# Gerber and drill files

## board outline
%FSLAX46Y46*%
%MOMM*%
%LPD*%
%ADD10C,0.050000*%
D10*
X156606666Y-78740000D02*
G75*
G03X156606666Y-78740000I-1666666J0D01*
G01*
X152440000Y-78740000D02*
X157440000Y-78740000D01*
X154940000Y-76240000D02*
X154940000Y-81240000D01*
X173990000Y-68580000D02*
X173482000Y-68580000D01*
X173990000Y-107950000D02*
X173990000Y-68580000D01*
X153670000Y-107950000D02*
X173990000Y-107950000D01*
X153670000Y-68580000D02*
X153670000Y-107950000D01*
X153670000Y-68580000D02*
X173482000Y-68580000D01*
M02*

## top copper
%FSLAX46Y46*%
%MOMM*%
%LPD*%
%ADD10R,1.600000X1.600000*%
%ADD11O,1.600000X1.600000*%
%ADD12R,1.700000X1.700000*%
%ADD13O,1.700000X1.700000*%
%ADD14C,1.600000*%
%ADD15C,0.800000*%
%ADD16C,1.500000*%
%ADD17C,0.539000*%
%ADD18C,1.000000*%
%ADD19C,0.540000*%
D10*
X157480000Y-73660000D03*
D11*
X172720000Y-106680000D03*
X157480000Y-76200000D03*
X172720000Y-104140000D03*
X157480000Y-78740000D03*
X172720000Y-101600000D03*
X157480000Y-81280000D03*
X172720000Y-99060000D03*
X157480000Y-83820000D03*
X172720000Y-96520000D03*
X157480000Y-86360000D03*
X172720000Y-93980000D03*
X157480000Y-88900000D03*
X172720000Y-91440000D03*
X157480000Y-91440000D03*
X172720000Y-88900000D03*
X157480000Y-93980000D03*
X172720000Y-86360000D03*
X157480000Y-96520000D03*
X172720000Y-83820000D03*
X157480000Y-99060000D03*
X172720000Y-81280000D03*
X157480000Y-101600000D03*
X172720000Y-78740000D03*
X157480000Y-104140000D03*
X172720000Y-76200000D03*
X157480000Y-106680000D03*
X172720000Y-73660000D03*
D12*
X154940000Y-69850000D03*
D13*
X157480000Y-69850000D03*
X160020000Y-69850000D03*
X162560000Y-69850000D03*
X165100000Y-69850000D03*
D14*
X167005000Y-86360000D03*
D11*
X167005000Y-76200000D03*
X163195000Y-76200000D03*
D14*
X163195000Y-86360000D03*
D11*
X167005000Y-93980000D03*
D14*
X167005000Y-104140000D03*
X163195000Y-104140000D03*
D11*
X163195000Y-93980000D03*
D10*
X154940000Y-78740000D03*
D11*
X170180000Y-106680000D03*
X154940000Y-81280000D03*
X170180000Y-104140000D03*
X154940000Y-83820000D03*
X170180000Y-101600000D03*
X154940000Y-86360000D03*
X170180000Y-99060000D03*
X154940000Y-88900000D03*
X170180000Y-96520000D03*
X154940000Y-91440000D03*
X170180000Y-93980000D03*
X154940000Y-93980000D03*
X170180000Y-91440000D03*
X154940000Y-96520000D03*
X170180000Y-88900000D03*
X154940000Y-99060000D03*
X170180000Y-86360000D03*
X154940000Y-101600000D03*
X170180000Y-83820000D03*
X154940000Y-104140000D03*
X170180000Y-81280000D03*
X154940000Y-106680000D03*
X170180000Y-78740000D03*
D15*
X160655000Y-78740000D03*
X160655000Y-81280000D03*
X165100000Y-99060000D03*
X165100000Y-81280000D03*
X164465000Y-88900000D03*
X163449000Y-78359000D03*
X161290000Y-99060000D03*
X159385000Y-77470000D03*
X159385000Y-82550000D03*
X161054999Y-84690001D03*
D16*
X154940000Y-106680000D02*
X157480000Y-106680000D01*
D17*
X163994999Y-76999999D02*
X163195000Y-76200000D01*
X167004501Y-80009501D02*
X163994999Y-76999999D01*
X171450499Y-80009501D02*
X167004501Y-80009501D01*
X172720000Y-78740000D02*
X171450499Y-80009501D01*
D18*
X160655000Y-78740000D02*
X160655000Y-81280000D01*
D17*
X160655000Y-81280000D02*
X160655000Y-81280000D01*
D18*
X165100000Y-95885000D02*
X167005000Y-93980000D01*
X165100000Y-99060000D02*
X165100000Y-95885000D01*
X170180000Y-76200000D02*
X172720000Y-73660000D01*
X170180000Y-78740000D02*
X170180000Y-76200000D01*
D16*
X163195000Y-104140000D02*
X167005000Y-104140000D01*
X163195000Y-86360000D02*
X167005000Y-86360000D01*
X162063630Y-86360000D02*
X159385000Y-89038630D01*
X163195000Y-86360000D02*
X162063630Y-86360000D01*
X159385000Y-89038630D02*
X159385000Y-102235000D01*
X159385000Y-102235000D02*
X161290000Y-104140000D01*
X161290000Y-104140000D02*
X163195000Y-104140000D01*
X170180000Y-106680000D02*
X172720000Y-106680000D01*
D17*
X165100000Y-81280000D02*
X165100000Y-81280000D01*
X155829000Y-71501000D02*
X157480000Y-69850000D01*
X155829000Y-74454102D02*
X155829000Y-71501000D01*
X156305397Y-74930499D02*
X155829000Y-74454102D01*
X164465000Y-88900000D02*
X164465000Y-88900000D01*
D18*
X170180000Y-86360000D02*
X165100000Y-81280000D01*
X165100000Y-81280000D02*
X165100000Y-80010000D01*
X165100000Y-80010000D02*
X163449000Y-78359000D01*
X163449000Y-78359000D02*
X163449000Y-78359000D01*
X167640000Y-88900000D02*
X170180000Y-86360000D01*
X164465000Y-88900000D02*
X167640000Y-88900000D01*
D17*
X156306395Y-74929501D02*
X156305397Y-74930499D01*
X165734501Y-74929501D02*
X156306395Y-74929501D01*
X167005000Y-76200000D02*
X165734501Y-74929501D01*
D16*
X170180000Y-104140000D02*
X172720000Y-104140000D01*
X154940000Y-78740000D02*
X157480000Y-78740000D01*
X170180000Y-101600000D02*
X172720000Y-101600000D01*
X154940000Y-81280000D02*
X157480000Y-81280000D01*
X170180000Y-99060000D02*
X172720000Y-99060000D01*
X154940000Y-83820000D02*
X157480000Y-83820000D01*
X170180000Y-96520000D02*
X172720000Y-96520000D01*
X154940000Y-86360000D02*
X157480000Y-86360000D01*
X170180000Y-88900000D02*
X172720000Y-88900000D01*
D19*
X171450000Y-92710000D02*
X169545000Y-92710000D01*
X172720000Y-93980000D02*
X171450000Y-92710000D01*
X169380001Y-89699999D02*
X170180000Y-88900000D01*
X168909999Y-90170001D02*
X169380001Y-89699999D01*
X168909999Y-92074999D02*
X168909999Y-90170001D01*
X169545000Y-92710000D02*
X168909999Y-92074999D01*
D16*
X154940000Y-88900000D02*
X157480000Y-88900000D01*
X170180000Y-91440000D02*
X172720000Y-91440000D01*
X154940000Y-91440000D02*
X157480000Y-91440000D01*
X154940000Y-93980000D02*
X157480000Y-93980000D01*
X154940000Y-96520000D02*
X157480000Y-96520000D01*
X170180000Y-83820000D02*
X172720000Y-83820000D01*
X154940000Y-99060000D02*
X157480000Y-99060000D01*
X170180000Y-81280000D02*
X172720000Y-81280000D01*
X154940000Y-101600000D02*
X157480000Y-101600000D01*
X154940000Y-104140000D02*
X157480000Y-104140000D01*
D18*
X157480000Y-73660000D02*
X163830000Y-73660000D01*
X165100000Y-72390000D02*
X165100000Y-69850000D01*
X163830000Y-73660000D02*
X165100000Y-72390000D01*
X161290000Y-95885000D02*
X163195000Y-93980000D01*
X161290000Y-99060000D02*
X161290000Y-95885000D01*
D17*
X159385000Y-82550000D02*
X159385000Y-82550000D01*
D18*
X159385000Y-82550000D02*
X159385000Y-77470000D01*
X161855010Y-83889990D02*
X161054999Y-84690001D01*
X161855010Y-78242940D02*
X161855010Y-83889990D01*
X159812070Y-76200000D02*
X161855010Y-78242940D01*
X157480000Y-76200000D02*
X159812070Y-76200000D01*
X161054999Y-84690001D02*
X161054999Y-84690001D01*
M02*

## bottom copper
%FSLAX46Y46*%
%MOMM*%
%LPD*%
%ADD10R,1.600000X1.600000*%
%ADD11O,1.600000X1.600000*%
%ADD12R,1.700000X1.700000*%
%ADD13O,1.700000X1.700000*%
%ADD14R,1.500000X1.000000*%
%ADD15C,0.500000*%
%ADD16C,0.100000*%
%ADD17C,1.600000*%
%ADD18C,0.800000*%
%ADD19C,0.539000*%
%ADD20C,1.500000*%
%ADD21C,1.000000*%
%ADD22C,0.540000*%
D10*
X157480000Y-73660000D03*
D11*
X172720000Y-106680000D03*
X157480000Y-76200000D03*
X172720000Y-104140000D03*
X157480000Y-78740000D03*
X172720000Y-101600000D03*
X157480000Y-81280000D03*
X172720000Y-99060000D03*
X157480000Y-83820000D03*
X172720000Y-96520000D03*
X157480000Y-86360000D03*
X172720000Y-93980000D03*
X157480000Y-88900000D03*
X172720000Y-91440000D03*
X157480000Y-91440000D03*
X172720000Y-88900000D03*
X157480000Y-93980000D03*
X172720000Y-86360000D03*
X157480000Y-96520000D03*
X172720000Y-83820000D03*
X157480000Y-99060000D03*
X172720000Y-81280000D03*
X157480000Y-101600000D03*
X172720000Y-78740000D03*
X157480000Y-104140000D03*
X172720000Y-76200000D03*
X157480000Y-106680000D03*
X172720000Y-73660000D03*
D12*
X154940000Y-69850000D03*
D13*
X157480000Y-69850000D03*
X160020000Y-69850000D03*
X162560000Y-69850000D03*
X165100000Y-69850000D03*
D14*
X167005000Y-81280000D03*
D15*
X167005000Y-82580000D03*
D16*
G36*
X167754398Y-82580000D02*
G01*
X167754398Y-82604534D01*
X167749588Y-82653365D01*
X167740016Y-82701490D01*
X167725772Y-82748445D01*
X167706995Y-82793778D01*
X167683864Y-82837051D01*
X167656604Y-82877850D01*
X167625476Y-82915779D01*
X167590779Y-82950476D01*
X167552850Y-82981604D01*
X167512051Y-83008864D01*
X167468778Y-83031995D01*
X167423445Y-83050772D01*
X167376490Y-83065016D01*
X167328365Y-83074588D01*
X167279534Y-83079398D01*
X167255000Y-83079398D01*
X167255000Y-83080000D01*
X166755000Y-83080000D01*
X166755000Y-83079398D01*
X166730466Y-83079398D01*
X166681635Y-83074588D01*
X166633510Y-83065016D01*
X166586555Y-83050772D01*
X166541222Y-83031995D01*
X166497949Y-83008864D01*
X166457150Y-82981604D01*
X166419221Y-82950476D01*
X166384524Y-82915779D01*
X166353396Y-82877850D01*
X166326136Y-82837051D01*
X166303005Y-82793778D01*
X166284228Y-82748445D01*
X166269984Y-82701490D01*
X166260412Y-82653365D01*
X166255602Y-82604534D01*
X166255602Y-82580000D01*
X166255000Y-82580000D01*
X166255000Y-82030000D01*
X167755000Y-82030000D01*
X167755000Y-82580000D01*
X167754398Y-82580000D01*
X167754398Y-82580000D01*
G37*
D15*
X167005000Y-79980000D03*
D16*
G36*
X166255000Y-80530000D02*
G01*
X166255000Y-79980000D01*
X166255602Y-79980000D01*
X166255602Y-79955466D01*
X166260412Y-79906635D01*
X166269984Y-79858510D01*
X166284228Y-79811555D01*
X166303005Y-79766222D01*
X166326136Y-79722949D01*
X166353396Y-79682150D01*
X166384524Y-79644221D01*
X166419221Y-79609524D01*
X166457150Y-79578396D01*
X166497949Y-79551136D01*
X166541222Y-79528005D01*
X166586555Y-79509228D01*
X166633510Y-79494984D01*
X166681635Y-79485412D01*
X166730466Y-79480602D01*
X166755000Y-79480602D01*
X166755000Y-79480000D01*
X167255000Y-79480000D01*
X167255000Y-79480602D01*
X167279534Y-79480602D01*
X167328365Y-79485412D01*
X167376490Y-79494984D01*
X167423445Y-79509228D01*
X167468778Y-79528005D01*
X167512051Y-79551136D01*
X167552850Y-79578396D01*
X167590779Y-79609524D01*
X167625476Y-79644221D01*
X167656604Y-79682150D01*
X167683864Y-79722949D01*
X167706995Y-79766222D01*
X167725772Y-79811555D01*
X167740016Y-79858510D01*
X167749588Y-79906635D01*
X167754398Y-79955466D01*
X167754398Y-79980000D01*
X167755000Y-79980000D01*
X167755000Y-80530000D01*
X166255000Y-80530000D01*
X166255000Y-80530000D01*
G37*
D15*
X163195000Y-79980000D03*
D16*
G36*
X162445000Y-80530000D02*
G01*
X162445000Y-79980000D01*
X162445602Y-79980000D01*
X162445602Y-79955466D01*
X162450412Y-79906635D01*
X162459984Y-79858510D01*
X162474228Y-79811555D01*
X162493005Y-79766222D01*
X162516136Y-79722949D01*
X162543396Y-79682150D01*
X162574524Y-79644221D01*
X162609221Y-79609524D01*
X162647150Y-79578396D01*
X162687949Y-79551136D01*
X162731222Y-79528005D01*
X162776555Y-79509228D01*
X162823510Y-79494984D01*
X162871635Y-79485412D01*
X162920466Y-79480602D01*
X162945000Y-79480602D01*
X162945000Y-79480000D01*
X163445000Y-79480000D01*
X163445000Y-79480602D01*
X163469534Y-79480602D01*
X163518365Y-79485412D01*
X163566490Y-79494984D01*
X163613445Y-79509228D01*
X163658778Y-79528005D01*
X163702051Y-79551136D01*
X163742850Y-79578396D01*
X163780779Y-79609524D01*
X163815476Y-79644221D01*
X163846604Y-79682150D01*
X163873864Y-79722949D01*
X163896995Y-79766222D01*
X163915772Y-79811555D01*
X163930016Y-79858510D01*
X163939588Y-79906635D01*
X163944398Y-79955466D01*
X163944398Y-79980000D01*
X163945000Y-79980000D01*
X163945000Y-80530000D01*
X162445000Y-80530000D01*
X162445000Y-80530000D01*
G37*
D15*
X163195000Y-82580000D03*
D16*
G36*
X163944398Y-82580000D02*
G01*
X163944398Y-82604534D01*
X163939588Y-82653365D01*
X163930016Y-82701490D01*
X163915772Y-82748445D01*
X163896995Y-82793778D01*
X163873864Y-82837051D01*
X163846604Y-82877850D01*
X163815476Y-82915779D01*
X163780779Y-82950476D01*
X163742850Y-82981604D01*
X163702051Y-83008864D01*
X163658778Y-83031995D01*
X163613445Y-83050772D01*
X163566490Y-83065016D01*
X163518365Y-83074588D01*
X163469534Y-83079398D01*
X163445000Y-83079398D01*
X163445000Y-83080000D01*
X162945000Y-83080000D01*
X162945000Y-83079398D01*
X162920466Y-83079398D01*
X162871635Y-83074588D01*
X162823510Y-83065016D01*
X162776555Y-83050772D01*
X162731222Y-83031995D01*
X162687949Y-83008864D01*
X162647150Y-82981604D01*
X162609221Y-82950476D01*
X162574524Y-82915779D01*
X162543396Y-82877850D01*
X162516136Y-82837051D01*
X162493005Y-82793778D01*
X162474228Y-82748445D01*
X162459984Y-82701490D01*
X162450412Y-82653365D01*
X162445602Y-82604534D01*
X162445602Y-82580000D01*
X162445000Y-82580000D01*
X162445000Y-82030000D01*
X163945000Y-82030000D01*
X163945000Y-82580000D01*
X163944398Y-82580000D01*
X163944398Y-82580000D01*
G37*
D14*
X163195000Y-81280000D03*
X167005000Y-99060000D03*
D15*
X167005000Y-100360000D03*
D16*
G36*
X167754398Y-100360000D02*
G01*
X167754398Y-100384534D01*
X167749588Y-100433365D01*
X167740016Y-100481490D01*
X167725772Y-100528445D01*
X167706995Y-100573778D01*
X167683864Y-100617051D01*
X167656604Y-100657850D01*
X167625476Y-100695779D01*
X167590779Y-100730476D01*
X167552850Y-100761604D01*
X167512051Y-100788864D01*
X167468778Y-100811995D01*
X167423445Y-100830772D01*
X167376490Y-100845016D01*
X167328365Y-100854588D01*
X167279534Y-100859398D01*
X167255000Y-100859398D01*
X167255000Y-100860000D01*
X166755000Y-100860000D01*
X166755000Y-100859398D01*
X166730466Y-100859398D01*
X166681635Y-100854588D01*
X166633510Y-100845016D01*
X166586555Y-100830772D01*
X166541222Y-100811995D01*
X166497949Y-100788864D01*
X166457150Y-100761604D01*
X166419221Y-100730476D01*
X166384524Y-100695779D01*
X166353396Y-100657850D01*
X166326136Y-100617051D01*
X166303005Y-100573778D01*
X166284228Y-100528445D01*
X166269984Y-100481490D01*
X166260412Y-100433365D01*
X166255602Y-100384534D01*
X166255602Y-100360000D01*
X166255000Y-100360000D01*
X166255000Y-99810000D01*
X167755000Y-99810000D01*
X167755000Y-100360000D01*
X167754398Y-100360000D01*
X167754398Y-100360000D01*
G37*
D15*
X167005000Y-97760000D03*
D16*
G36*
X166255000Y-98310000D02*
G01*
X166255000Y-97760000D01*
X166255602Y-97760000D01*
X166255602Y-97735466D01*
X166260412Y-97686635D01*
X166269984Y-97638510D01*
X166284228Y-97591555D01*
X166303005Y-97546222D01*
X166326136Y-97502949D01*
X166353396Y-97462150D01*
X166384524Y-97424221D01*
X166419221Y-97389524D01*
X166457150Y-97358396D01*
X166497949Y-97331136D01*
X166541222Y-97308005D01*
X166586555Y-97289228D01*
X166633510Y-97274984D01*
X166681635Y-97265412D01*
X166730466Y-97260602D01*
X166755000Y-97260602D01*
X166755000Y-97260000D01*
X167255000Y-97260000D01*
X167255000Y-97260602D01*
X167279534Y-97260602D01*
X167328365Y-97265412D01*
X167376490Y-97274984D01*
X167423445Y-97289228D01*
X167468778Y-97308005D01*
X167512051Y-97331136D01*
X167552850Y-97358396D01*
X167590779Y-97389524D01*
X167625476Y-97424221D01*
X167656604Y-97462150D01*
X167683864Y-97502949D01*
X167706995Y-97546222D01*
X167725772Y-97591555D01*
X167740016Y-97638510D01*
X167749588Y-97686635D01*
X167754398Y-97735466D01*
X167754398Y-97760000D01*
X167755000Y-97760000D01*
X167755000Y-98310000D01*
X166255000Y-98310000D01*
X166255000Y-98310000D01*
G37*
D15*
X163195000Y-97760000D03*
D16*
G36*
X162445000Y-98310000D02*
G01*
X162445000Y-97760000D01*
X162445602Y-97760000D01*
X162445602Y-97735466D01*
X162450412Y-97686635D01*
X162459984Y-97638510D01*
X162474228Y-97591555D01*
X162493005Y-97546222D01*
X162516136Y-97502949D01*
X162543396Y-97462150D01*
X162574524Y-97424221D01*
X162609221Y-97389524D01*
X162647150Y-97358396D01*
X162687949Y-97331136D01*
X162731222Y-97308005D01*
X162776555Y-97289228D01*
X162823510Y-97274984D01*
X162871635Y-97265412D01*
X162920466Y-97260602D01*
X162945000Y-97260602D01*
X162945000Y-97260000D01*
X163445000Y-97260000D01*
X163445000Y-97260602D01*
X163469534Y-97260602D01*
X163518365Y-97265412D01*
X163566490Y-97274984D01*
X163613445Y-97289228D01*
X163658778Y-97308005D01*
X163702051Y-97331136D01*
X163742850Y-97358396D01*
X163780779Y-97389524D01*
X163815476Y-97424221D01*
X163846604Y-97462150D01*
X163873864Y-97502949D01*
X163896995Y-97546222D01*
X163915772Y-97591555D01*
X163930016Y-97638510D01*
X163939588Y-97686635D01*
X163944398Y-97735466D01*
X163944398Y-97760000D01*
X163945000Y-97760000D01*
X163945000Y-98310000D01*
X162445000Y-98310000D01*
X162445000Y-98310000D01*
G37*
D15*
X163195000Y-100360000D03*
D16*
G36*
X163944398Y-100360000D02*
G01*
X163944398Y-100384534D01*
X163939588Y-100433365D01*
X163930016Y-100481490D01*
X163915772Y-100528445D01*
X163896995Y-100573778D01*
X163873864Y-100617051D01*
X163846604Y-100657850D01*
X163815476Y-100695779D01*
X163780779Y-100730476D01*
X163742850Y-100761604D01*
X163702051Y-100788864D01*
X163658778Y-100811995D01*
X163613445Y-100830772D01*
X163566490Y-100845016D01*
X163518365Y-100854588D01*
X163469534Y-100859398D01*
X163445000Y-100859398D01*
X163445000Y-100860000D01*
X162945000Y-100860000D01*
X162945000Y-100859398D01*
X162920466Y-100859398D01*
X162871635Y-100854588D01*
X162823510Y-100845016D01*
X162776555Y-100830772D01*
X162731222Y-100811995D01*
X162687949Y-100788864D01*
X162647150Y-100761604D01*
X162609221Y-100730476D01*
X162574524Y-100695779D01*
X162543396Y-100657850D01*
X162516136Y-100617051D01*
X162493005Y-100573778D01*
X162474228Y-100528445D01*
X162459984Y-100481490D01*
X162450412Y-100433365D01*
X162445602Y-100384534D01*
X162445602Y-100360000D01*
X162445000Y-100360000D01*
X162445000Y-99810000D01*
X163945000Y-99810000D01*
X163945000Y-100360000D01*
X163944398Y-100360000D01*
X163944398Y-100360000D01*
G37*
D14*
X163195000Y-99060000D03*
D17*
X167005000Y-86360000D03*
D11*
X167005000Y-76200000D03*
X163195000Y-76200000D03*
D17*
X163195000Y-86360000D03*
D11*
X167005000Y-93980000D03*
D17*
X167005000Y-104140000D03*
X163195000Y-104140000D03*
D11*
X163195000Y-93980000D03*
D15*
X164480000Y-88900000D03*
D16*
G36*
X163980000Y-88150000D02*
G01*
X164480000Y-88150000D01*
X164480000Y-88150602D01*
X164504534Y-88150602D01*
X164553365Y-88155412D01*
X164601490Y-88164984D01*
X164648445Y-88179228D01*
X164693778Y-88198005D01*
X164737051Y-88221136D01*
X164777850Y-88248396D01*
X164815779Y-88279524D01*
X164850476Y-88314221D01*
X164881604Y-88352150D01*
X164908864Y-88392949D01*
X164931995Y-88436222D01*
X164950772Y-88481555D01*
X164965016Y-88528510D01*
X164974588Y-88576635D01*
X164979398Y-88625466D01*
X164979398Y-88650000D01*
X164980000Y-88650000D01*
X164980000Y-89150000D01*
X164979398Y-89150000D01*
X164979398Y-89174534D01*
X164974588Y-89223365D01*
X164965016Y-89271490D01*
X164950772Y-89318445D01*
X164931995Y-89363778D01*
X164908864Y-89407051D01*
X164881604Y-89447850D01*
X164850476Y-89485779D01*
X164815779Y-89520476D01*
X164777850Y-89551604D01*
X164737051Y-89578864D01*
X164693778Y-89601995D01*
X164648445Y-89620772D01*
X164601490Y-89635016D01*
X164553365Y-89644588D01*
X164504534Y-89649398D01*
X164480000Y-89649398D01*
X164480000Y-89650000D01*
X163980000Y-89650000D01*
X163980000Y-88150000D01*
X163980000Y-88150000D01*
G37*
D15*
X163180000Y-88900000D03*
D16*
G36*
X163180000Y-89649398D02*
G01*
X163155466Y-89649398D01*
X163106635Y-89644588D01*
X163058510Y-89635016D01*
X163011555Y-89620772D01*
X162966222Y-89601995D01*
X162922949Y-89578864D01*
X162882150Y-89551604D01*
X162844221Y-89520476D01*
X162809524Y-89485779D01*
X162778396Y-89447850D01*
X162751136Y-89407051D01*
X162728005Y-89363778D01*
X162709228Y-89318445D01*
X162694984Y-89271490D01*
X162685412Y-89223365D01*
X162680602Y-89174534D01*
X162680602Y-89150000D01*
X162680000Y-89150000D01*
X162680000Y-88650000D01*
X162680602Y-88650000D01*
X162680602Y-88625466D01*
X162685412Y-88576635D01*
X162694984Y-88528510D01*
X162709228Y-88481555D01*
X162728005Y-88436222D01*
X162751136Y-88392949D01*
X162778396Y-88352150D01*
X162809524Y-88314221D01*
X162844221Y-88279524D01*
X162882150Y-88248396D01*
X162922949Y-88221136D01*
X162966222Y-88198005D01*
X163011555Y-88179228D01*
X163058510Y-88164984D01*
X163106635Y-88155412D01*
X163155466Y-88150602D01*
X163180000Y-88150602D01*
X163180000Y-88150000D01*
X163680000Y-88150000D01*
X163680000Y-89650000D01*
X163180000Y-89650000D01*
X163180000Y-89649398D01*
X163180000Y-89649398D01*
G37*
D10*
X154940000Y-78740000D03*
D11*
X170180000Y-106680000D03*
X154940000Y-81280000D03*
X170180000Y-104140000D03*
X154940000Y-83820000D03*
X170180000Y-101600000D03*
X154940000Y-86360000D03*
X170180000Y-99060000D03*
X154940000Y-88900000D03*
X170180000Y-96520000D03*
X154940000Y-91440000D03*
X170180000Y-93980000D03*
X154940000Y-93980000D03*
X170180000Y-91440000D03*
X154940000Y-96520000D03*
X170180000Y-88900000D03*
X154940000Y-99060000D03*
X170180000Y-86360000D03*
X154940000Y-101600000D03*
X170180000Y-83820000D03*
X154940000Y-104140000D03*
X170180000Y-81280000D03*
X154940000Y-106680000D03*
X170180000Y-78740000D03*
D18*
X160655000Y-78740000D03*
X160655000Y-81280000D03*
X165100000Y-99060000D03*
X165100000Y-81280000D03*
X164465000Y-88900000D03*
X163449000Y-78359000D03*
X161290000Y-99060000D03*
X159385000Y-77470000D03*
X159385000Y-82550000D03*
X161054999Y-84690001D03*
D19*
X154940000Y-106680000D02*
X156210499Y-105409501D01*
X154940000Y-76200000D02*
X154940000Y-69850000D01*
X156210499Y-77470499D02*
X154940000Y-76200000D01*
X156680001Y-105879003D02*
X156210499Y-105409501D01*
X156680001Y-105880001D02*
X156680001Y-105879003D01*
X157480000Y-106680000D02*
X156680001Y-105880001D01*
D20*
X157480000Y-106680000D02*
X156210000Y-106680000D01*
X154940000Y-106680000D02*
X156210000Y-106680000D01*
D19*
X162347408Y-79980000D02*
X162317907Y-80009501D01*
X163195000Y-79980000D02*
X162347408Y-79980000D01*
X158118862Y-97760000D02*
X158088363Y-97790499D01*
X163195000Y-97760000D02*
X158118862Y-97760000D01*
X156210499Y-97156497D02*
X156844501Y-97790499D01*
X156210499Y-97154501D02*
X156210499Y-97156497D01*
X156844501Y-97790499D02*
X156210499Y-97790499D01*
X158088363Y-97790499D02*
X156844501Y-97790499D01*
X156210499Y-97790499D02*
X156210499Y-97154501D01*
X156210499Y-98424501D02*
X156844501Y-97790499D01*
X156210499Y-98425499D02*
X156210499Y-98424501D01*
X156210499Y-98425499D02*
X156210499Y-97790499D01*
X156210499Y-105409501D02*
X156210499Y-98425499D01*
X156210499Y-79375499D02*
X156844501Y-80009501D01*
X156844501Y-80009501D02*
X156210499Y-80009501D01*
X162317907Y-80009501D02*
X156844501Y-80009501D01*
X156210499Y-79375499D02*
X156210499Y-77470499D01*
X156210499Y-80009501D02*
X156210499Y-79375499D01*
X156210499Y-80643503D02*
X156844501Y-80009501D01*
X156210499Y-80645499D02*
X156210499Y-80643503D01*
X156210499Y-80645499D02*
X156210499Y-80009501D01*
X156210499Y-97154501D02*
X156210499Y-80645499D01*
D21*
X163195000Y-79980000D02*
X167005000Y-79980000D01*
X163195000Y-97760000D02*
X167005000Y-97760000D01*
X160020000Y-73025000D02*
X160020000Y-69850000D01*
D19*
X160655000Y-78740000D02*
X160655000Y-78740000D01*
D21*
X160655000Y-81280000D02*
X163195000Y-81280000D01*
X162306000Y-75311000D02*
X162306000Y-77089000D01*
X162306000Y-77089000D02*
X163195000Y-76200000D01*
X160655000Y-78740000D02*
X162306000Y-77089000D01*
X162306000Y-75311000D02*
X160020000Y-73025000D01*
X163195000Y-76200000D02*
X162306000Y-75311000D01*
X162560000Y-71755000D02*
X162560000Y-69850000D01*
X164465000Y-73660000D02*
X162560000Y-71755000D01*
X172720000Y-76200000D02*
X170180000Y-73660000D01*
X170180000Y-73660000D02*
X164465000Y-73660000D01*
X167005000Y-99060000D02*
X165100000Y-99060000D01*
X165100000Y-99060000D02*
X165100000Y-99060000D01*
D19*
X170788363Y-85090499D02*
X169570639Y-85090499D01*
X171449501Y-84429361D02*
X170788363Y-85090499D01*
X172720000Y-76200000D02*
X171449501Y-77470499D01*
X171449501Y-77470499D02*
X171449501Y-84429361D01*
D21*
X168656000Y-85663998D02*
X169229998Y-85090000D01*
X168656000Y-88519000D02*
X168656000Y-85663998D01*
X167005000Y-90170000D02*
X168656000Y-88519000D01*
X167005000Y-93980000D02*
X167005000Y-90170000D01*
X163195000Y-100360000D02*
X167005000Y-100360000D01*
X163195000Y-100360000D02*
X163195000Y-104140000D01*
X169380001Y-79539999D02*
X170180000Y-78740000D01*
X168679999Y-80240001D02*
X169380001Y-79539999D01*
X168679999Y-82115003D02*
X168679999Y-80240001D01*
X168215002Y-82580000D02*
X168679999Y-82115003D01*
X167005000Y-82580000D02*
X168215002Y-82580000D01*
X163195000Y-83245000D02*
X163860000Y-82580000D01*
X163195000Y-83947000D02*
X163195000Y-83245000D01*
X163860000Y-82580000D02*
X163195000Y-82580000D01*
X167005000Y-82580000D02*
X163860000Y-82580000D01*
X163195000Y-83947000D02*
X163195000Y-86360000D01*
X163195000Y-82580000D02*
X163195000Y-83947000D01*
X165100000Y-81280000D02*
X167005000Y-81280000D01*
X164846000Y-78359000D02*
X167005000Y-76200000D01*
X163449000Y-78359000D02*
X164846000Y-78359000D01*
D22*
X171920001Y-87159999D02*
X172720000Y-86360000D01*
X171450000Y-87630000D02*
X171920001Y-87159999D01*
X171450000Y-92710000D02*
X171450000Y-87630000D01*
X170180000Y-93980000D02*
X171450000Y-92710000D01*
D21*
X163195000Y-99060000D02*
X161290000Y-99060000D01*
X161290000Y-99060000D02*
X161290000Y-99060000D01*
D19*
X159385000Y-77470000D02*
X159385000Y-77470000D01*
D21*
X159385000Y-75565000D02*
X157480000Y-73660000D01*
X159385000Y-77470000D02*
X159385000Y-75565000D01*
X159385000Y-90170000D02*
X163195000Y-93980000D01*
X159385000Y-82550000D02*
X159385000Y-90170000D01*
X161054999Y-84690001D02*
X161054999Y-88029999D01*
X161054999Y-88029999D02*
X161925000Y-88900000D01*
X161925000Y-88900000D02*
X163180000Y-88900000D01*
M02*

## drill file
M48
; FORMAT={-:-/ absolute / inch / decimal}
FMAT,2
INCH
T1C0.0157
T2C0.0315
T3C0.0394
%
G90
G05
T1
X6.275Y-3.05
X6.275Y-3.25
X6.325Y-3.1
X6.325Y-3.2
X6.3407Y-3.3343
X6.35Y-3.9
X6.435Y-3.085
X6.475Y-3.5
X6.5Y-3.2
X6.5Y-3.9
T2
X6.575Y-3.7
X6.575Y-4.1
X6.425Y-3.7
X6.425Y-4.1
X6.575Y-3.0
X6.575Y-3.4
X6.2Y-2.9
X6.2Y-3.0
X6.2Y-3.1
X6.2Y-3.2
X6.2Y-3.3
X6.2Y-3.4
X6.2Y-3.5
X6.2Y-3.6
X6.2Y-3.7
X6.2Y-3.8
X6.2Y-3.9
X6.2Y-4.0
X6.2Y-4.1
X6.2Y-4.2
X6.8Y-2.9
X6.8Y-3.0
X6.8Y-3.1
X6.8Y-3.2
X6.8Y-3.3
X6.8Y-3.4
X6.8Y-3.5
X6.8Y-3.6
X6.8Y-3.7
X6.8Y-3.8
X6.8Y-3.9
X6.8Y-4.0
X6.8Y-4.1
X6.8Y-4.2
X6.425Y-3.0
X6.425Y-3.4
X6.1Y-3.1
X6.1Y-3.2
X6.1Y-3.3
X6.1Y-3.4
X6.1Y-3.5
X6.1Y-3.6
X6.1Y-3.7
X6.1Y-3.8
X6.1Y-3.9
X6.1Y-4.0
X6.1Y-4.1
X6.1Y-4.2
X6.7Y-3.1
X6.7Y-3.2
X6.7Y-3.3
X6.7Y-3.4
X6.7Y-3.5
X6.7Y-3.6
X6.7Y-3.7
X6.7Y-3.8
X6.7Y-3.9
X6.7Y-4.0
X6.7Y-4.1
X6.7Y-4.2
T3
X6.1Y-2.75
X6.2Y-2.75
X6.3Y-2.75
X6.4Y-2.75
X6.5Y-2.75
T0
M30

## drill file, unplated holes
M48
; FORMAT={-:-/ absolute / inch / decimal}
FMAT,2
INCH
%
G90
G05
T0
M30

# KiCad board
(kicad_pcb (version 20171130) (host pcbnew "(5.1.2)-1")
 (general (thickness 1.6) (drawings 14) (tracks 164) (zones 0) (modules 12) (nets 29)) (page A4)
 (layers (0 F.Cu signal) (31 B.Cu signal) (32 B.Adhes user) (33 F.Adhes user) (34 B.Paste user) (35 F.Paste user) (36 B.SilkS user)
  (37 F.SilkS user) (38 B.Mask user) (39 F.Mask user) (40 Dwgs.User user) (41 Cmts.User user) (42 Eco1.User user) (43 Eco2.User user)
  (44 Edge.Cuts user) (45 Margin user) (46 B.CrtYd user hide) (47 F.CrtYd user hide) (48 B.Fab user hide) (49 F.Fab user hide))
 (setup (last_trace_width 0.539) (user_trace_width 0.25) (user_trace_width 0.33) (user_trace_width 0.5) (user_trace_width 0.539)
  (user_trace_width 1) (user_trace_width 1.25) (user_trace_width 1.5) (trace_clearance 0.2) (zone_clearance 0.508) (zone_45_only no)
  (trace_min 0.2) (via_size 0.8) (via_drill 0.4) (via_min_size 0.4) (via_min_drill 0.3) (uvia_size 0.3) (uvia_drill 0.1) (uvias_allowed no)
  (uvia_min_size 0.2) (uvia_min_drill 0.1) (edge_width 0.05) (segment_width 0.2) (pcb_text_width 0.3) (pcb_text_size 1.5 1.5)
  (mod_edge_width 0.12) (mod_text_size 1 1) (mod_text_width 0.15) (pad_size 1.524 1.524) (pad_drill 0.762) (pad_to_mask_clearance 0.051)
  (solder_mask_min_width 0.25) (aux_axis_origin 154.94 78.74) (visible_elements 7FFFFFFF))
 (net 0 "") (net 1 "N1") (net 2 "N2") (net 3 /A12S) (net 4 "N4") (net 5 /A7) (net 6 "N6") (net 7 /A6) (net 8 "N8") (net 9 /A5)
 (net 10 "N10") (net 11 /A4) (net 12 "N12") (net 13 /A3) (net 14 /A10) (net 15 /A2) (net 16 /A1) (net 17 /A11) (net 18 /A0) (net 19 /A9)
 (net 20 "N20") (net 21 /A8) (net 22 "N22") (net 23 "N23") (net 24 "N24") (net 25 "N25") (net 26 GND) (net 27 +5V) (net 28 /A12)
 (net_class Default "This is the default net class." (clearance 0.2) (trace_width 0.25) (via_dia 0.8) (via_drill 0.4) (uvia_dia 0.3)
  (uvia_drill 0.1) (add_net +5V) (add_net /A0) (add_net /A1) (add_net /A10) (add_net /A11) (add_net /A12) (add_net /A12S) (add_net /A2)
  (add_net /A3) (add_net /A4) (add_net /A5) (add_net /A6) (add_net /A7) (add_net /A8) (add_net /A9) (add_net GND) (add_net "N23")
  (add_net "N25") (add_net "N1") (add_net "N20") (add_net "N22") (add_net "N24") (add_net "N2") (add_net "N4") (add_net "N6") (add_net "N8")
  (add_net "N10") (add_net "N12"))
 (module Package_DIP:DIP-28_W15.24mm (layer F.Cu) (at 157.48 73.66)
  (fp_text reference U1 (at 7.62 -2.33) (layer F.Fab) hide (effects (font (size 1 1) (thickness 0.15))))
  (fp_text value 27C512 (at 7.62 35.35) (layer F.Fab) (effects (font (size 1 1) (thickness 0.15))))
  (pad 1 thru_hole rect (at 0 0) (size 1.6 1.6) (drill 0.8) (layers *.Cu *.Mask) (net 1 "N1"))
  (pad 15 thru_hole oval (at 15.24 33.02) (size 1.6 1.6) (drill 0.8) (layers *.Cu *.Mask) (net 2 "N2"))
  (pad 2 thru_hole oval (at 0 2.54) (size 1.6 1.6) (drill 0.8) (layers *.Cu *.Mask) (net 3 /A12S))
  (pad 16 thru_hole oval (at 15.24 30.48) (size 1.6 1.6) (drill 0.8) (layers *.Cu *.Mask) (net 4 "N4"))
  (pad 3 thru_hole oval (at 0 5.08) (size 1.6 1.6) (drill 0.8) (layers *.Cu *.Mask) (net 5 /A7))
  (pad 17 thru_hole oval (at 15.24 27.94) (size 1.6 1.6) (drill 0.8) (layers *.Cu *.Mask) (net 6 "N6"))
  (pad 4 thru_hole oval (at 0 7.62) (size 1.6 1.6) (drill 0.8) (layers *.Cu *.Mask) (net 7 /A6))
  (pad 18 thru_hole oval (at 15.24 25.4) (size 1.6 1.6) (drill 0.8) (layers *.Cu *.Mask) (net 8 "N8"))
  (pad 5 thru_hole oval (at 0 10.16) (size 1.6 1.6) (drill 0.8) (layers *.Cu *.Mask) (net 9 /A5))
  (pad 19 thru_hole oval (at 15.24 22.86) (size 1.6 1.6) (drill 0.8) (layers *.Cu *.Mask) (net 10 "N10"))
  (pad 6 thru_hole oval (at 0 12.7) (size 1.6 1.6) (drill 0.8) (layers *.Cu *.Mask) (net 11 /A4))
  (pad 20 thru_hole oval (at 15.24 20.32) (size 1.6 1.6) (drill 0.8) (layers *.Cu *.Mask) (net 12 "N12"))
  (pad 7 thru_hole oval (at 0 15.24) (size 1.6 1.6) (drill 0.8) (layers *.Cu *.Mask) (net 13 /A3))
  (pad 21 thru_hole oval (at 15.24 17.78) (size 1.6 1.6) (drill 0.8) (layers *.Cu *.Mask) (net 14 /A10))
  (pad 8 thru_hole oval (at 0 17.78) (size 1.6 1.6) (drill 0.8) (layers *.Cu *.Mask) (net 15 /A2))
  (pad 22 thru_hole oval (at 15.24 15.24) (size 1.6 1.6) (drill 0.8) (layers *.Cu *.Mask) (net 12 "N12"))
  (pad 9 thru_hole oval (at 0 20.32) (size 1.6 1.6) (drill 0.8) (layers *.Cu *.Mask) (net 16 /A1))
  (pad 23 thru_hole oval (at 15.24 12.7) (size 1.6 1.6) (drill 0.8) (layers *.Cu *.Mask) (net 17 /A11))
  (pad 10 thru_hole oval (at 0 22.86) (size 1.6 1.6) (drill 0.8) (layers *.Cu *.Mask) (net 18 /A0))
  (pad 24 thru_hole oval (at 15.24 10.16) (size 1.6 1.6) (drill 0.8) (layers *.Cu *.Mask) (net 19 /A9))
  (pad 11 thru_hole oval (at 0 25.4) (size 1.6 1.6) (drill 0.8) (layers *.Cu *.Mask) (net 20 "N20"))
  (pad 25 thru_hole oval (at 15.24 7.62) (size 1.6 1.6) (drill 0.8) (layers *.Cu *.Mask) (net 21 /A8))
  (pad 12 thru_hole oval (at 0 27.94) (size 1.6 1.6) (drill 0.8) (layers *.Cu *.Mask) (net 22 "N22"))
  (pad 26 thru_hole oval (at 15.24 5.08) (size 1.6 1.6) (drill 0.8) (layers *.Cu *.Mask) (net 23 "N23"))
  (pad 13 thru_hole oval (at 0 30.48) (size 1.6 1.6) (drill 0.8) (layers *.Cu *.Mask) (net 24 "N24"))
  (pad 27 thru_hole oval (at 15.24 2.54) (size 1.6 1.6) (drill 0.8) (layers *.Cu *.Mask) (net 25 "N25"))
  (pad 14 thru_hole oval (at 0 33.02) (size 1.6 1.6) (drill 0.8) (layers *.Cu *.Mask) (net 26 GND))
  (pad 28 thru_hole oval (at 15.24 0) (size 1.6 1.6) (drill 0.8) (layers *.Cu *.Mask) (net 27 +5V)))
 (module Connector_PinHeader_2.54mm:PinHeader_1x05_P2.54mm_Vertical (layer F.Cu) (at 154.94 69.85 90)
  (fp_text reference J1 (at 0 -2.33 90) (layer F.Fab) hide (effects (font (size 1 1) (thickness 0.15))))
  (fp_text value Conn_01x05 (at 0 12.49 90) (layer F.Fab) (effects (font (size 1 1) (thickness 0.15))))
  (pad 1 thru_hole rect (at 0 0 90) (size 1.7 1.7) (drill 1) (layers *.Cu *.Mask) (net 26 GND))
  (pad 2 thru_hole oval (at 0 2.54 90) (size 1.7 1.7) (drill 1) (layers *.Cu *.Mask) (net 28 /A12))
  (pad 3 thru_hole oval (at 0 5.08 90) (size 1.7 1.7) (drill 1) (layers *.Cu *.Mask) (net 23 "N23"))
  (pad 4 thru_hole oval (at 0 7.62 90) (size 1.7 1.7) (drill 1) (layers *.Cu *.Mask) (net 25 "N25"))
  (pad 5 thru_hole oval (at 0 10.16 90) (size 1.7 1.7) (drill 1) (layers *.Cu *.Mask) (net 1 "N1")))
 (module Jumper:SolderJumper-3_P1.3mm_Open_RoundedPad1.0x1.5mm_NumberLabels (layer B.Cu) (at 167.005 81.28 270)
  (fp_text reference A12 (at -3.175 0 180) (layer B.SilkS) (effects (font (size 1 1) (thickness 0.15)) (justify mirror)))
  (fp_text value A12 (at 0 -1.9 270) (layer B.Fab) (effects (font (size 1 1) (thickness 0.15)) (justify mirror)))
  (pad 2 smd rect (at 0 0 270) (size 1 1.5) (layers B.Cu B.Mask) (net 28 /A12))
  (pad 3 smd custom (at 1.3 0 270) (size 1 0.5) (layers B.Cu B.Mask) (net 27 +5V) (zone_connect 2)
   (options (clearance outline) (anchor rect)) (primitives))
  (pad 1 smd custom (at -1.3 0 270) (size 1 0.5) (layers B.Cu B.Mask) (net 26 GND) (zone_connect 2)
   (options (clearance outline) (anchor rect)) (primitives)))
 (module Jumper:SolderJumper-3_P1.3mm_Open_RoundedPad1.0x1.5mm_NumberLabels (layer B.Cu) (at 163.195 81.28 270)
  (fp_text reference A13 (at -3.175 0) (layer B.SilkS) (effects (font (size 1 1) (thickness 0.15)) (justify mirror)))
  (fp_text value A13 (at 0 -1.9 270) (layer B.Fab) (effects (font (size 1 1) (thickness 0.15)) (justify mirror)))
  (pad 1 smd custom (at -1.3 0 270) (size 1 0.5) (layers B.Cu B.Mask) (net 26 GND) (zone_connect 2)
   (options (clearance outline) (anchor rect)) (primitives))
  (pad 3 smd custom (at 1.3 0 270) (size 1 0.5) (layers B.Cu B.Mask) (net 27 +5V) (zone_connect 2)
   (options (clearance outline) (anchor rect)) (primitives))
  (pad 2 smd rect (at 0 0 270) (size 1 1.5) (layers B.Cu B.Mask) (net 23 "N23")))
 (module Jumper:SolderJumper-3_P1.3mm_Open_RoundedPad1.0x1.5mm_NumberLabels (layer B.Cu) (at 167.005 99.06 270)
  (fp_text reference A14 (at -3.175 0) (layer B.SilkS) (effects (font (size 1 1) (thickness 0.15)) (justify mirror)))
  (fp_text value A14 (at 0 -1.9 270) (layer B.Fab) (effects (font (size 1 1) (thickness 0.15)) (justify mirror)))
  (pad 2 smd rect (at 0 0 270) (size 1 1.5) (layers B.Cu B.Mask) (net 25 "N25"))
  (pad 3 smd custom (at 1.3 0 270) (size 1 0.5) (layers B.Cu B.Mask) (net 27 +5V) (zone_connect 2)
   (options (clearance outline) (anchor rect)) (primitives))
  (pad 1 smd custom (at -1.3 0 270) (size 1 0.5) (layers B.Cu B.Mask) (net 26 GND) (zone_connect 2)
   (options (clearance outline) (anchor rect)) (primitives)))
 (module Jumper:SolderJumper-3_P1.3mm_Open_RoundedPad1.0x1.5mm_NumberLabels (layer B.Cu) (at 163.195 99.06 270)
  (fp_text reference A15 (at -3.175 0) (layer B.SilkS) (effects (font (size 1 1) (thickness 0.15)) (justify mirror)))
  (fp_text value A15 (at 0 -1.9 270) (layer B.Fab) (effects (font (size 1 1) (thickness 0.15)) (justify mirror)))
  (pad 1 smd custom (at -1.3 0 270) (size 1 0.5) (layers B.Cu B.Mask) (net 26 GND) (zone_connect 2)
   (options (clearance outline) (anchor rect)) (primitives))
  (pad 3 smd custom (at 1.3 0 270) (size 1 0.5) (layers B.Cu B.Mask) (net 27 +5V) (zone_connect 2)
   (options (clearance outline) (anchor rect)) (primitives))
  (pad 2 smd rect (at 0 0 270) (size 1 1.5) (layers B.Cu B.Mask) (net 1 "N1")))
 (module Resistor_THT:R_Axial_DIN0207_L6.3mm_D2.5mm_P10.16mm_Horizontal (layer F.Cu) (at 167.005 86.36 90)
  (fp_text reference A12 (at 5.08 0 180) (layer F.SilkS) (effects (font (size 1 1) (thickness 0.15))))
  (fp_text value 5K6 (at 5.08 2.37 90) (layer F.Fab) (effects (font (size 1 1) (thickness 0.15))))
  (pad 1 thru_hole circle (at 0 0 90) (size 1.6 1.6) (drill 0.8) (layers *.Cu *.Mask) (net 27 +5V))
  (pad 2 thru_hole oval (at 10.16 0 90) (size 1.6 1.6) (drill 0.8) (layers *.Cu *.Mask) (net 28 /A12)))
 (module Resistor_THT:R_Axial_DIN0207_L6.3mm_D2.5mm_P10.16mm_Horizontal (layer F.Cu) (at 163.195 86.36 90)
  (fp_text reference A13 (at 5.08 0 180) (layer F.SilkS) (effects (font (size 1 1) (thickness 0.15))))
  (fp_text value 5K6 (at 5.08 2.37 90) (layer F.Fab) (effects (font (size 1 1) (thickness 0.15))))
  (pad 2 thru_hole oval (at 10.16 0 90) (size 1.6 1.6) (drill 0.8) (layers *.Cu *.Mask) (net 23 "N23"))
  (pad 1 thru_hole circle (at 0 0 90) (size 1.6 1.6) (drill 0.8) (layers *.Cu *.Mask) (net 27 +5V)))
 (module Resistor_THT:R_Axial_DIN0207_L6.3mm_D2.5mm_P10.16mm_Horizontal (layer F.Cu) (at 167.005 104.14 90)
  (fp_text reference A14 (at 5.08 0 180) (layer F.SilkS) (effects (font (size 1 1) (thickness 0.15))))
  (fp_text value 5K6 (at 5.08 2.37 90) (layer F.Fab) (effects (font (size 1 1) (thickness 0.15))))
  (pad 2 thru_hole oval (at 10.16 0 90) (size 1.6 1.6) (drill 0.8) (layers *.Cu *.Mask) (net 25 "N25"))
  (pad 1 thru_hole circle (at 0 0 90) (size 1.6 1.6) (drill 0.8) (layers *.Cu *.Mask) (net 27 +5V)))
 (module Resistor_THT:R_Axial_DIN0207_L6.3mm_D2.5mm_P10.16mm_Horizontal (layer F.Cu) (at 163.195 104.14 90)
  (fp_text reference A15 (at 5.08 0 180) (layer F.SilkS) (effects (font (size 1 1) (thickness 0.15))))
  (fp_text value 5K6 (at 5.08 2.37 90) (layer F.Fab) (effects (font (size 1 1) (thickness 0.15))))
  (pad 1 thru_hole circle (at 0 0 90) (size 1.6 1.6) (drill 0.8) (layers *.Cu *.Mask) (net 27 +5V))
  (pad 2 thru_hole oval (at 10.16 0 90) (size 1.6 1.6) (drill 0.8) (layers *.Cu *.Mask) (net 1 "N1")))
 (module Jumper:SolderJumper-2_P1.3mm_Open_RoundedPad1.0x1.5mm (layer B.Cu) (at 163.83 88.9 180)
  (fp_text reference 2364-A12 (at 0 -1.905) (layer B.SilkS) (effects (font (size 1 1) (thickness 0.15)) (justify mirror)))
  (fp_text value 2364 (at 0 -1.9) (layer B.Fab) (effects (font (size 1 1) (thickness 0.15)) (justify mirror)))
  (pad 1 smd custom (at -0.65 0 180) (size 1 0.5) (layers B.Cu B.Mask) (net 28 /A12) (zone_connect 2)
   (options (clearance outline) (anchor rect)) (primitives))
  (pad 2 smd custom (at 0.65 0 180) (size 1 0.5) (layers B.Cu B.Mask) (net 3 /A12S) (zone_connect 2)
   (options (clearance outline) (anchor rect)) (primitives)))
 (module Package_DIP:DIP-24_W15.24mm (layer F.Cu) (at 154.94 78.74)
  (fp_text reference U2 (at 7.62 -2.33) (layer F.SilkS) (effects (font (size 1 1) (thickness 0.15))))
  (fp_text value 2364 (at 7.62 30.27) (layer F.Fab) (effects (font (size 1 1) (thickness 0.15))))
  (pad 1 thru_hole rect (at 0 0) (size 1.6 1.6) (drill 0.8) (layers *.Cu *.Mask) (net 5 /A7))
  (pad 13 thru_hole oval (at 15.24 27.94) (size 1.6 1.6) (drill 0.8) (layers *.Cu *.Mask) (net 2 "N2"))
  (pad 2 thru_hole oval (at 0 2.54) (size 1.6 1.6) (drill 0.8) (layers *.Cu *.Mask) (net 7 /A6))
  (pad 14 thru_hole oval (at 15.24 25.4) (size 1.6 1.6) (drill 0.8) (layers *.Cu *.Mask) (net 4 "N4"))
  (pad 3 thru_hole oval (at 0 5.08) (size 1.6 1.6) (drill 0.8) (layers *.Cu *.Mask) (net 9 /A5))
  (pad 15 thru_hole oval (at 15.24 22.86) (size 1.6 1.6) (drill 0.8) (layers *.Cu *.Mask) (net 6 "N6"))
  (pad 4 thru_hole oval (at 0 7.62) (size 1.6 1.6) (drill 0.8) (layers *.Cu *.Mask) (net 11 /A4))
  (pad 16 thru_hole oval (at 15.24 20.32) (size 1.6 1.6) (drill 0.8) (layers *.Cu *.Mask) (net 8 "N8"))
  (pad 5 thru_hole oval (at 0 10.16) (size 1.6 1.6) (drill 0.8) (layers *.Cu *.Mask) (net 13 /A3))
  (pad 17 thru_hole oval (at 15.24 17.78) (size 1.6 1.6) (drill 0.8) (layers *.Cu *.Mask) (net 10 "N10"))
  (pad 6 thru_hole oval (at 0 12.7) (size 1.6 1.6) (drill 0.8) (layers *.Cu *.Mask) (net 15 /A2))
  (pad 18 thru_hole oval (at 15.24 15.24) (size 1.6 1.6) (drill 0.8) (layers *.Cu *.Mask) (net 17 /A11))
  (pad 7 thru_hole oval (at 0 15.24) (size 1.6 1.6) (drill 0.8) (layers *.Cu *.Mask) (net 16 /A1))
  (pad 19 thru_hole oval (at 15.24 12.7) (size 1.6 1.6) (drill 0.8) (layers *.Cu *.Mask) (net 14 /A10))
  (pad 8 thru_hole oval (at 0 17.78) (size 1.6 1.6) (drill 0.8) (layers *.Cu *.Mask) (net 18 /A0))
  (pad 20 thru_hole oval (at 15.24 10.16) (size 1.6 1.6) (drill 0.8) (layers *.Cu *.Mask) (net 12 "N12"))
  (pad 9 thru_hole oval (at 0 20.32) (size 1.6 1.6) (drill 0.8) (layers *.Cu *.Mask) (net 20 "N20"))
  (pad 21 thru_hole oval (at 15.24 7.62) (size 1.6 1.6) (drill 0.8) (layers *.Cu *.Mask) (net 28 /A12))
  (pad 10 thru_hole oval (at 0 22.86) (size 1.6 1.6) (drill 0.8) (layers *.Cu *.Mask) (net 22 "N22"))
  (pad 22 thru_hole oval (at 15.24 5.08) (size 1.6 1.6) (drill 0.8) (layers *.Cu *.Mask) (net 19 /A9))
  (pad 11 thru_hole oval (at 0 25.4) (size 1.6 1.6) (drill 0.8) (layers *.Cu *.Mask) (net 24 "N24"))
  (pad 23 thru_hole oval (at 15.24 2.54) (size 1.6 1.6) (drill 0.8) (layers *.Cu *.Mask) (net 21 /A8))
  (pad 12 thru_hole oval (at 0 27.94) (size 1.6 1.6) (drill 0.8) (layers *.Cu *.Mask) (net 26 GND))
  (pad 24 thru_hole oval (at 15.24 0) (size 1.6 1.6) (drill 0.8) (layers *.Cu *.Mask) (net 27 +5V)))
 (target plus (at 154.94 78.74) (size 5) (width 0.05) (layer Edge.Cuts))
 (gr_line (start 173.99 68.58) (end 173.482 68.58) (layer Edge.Cuts) (width 0.05))
 (gr_line (start 173.99 107.95) (end 173.99 68.58) (layer Edge.Cuts) (width 0.05))
 (gr_line (start 153.67 107.95) (end 173.99 107.95) (layer Edge.Cuts) (width 0.05))
 (gr_line (start 153.67 68.58) (end 153.67 107.95) (layer Edge.Cuts) (width 0.05))
 (gr_line (start 153.67 68.58) (end 173.482 68.58) (layer Edge.Cuts) (width 0.05))
 (segment (start 154.94 106.68) (end 157.48 106.68) (width 1.5) (layer F.Cu) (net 26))
 (segment (start 154.94 106.68) (end 156.210499 105.409501) (width 0.539) (layer B.Cu) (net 26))
 (segment (start 154.94 76.2) (end 154.94 69.85) (width 0.539) (layer B.Cu) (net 26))
 (segment (start 156.210499 77.470499) (end 154.94 76.2) (width 0.539) (layer B.Cu) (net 26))
 (segment (start 156.680001 105.879003) (end 156.210499 105.409501) (width 0.539) (layer B.Cu) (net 26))
 (segment (start 156.680001 105.880001) (end 156.680001 105.879003) (width 0.539) (layer B.Cu) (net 26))
 (segment (start 157.48 106.68) (end 156.680001 105.880001) (width 0.539) (layer B.Cu) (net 26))
 (segment (start 157.48 106.68) (end 156.21 106.68) (width 1.5) (layer B.Cu) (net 26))
 (segment (start 154.94 106.68) (end 156.21 106.68) (width 1.5) (layer B.Cu) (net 26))
 (segment (start 162.347408 79.98) (end 162.317907 80.009501) (width 0.539) (layer B.Cu) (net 26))
 (segment (start 163.195 79.98) (end 162.347408 79.98) (width 0.539) (layer B.Cu) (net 26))
 (segment (start 158.118862 97.76) (end 158.088363 97.790499) (width 0.539) (layer B.Cu) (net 26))
 (segment (start 163.195 97.76) (end 158.118862 97.76) (width 0.539) (layer B.Cu) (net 26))
 (segment (start 156.210499 97.156497) (end 156.844501 97.790499) (width 0.539) (layer B.Cu) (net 26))
 (segment (start 156.210499 97.154501) (end 156.210499 97.156497) (width 0.539) (layer B.Cu) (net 26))
 (segment (start 156.844501 97.790499) (end 156.210499 97.790499) (width 0.539) (layer B.Cu) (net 26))
 (segment (start 158.088363 97.790499) (end 156.844501 97.790499) (width 0.539) (layer B.Cu) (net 26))
 (segment (start 156.210499 97.790499) (end 156.210499 97.154501) (width 0.539) (layer B.Cu) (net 26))
 (segment (start 156.210499 98.424501) (end 156.844501 97.790499) (width 0.539) (layer B.Cu) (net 26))
 (segment (start 156.210499 98.425499) (end 156.210499 98.424501) (width 0.539) (layer B.Cu) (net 26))
 (segment (start 156.210499 98.425499) (end 156.210499 97.790499) (width 0.539) (layer B.Cu) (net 26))
 (segment (start 156.210499 105.409501) (end 156.210499 98.425499) (width 0.539) (layer B.Cu) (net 26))
 (segment (start 156.210499 79.375499) (end 156.844501 80.009501) (width 0.539) (layer B.Cu) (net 26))
 (segment (start 156.844501 80.009501) (end 156.210499 80.009501) (width 0.539) (layer B.Cu) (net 26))
 (segment (start 162.317907 80.009501) (end 156.844501 80.009501) (width 0.539) (layer B.Cu) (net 26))
 (segment (start 156.210499 79.375499) (end 156.210499 77.470499) (width 0.539) (layer B.Cu) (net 26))
 (segment (start 156.210499 80.009501) (end 156.210499 79.375499) (width 0.539) (layer B.Cu) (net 26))
 (segment (start 156.210499 80.643503) (end 156.844501 80.009501) (width 0.539) (layer B.Cu) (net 26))
 (segment (start 156.210499 80.645499) (end 156.210499 80.643503) (width 0.539) (layer B.Cu) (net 26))
 (segment (start 156.210499 80.645499) (end 156.210499 80.009501) (width 0.539) (layer B.Cu) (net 26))
 (segment (start 156.210499 97.154501) (end 156.210499 80.645499) (width 0.539) (layer B.Cu) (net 26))
 (segment (start 163.195 79.98) (end 167.005 79.98) (width 1) (layer B.Cu) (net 26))
 (segment (start 163.195 97.76) (end 167.005 97.76) (width 1) (layer B.Cu) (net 26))
 (segment (start 163.994999 76.999999) (end 163.195 76.2) (width 0.539) (layer F.Cu) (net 23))
 (segment (start 167.004501 80.009501) (end 163.994999 76.999999) (width 0.539) (layer F.Cu) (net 23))
 (segment (start 171.450499 80.009501) (end 167.004501 80.009501) (width 0.539) (layer F.Cu) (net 23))
 (segment (start 172.72 78.74) (end 171.450499 80.009501) (width 0.539) (layer F.Cu) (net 23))
 (segment (start 160.02 73.025) (end 160.02 69.85) (width 1) (layer B.Cu) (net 23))
 (segment (start 160.655 78.74) (end 160.655 78.74) (width 0.539) (layer B.Cu) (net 23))
 (via (at 160.655 78.74) (size 0.8) (drill 0.4) (layers F.Cu B.Cu) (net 23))
 (segment (start 160.655 78.74) (end 160.655 81.28) (width 1) (layer F.Cu) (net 23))
 (segment (start 160.655 81.28) (end 160.655 81.28) (width 0.539) (layer F.Cu) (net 23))
 (via (at 160.655 81.28) (size 0.8) (drill 0.4) (layers F.Cu B.Cu) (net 23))
 (segment (start 160.655 81.28) (end 163.195 81.28) (width 1) (layer B.Cu) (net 23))
 (segment (start 162.306 75.311) (end 162.306 77.089) (width 1) (layer B.Cu) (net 23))
 (segment (start 162.306 77.089) (end 163.195 76.2) (width 1) (layer B.Cu) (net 23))
 (segment (start 160.655 78.74) (end 162.306 77.089) (width 1) (layer B.Cu) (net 23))
 (segment (start 162.306 75.311) (end 160.02 73.025) (width 1) (layer B.Cu) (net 23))
 (segment (start 163.195 76.2) (end 162.306 75.311) (width 1) (layer B.Cu) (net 23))
 (segment (start 162.56 71.755) (end 162.56 69.85) (width 1) (layer B.Cu) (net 25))
 (segment (start 164.465 73.66) (end 162.56 71.755) (width 1) (layer B.Cu) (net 25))
 (segment (start 172.72 76.2) (end 170.18 73.66) (width 1) (layer B.Cu) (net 25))
 (segment (start 170.18 73.66) (end 164.465 73.66) (width 1) (layer B.Cu) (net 25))
 (segment (start 167.005 99.06) (end 165.1 99.06) (width 1) (layer B.Cu) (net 25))
 (segment (start 165.1 99.06) (end 165.1 99.06) (width 1) (layer B.Cu) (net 25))
 (via (at 165.1 99.06) (size 0.8) (drill 0.4) (layers F.Cu B.Cu) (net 25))
 (segment (start 165.1 95.885) (end 167.005 93.98) (width 1) (layer F.Cu) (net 25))
 (segment (start 165.1 99.06) (end 165.1 95.885) (width 1) (layer F.Cu) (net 25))
 (segment (start 170.788363 85.090499) (end 169.570639 85.090499) (width 0.539) (layer B.Cu) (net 25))
 (segment (start 171.449501 84.429361) (end 170.788363 85.090499) (width 0.539) (layer B.Cu) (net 25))
 (segment (start 172.72 76.2) (end 171.449501 77.470499) (width 0.539) (layer B.Cu) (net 25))
 (segment (start 171.449501 77.470499) (end 171.449501 84.429361) (width 0.539) (layer B.Cu) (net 25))
 (segment (start 168.656 85.663998) (end 169.229998 85.09) (width 1) (layer B.Cu) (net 25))
 (segment (start 168.656 88.519) (end 168.656 85.663998) (width 1) (layer B.Cu) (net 25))
 (segment (start 167.005 90.17) (end 168.656 88.519) (width 1) (layer B.Cu) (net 25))
 (segment (start 167.005 93.98) (end 167.005 90.17) (width 1) (layer B.Cu) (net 25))
 (segment (start 170.18 76.2) (end 172.72 73.66) (width 1) (layer F.Cu) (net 27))
 (segment (start 170.18 78.74) (end 170.18 76.2) (width 1) (layer F.Cu) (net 27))
 (segment (start 163.195 104.14) (end 167.005 104.14) (width 1.5) (layer F.Cu) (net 27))
 (segment (start 163.195 86.36) (end 167.005 86.36) (width 1.5) (layer F.Cu) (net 27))
 (segment (start 163.195 100.36) (end 167.005 100.36) (width 1) (layer B.Cu) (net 27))
 (segment (start 163.195 100.36) (end 163.195 104.14) (width 1) (layer B.Cu) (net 27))
 (segment (start 169.380001 79.539999) (end 170.18 78.74) (width 1) (layer B.Cu) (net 27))
 (segment (start 168.679999 80.240001) (end 169.380001 79.539999) (width 1) (layer B.Cu) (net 27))
 (segment (start 168.679999 82.115003) (end 168.679999 80.240001) (width 1) (layer B.Cu) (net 27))
 (segment (start 168.215002 82.58) (end 168.679999 82.115003) (width 1) (layer B.Cu) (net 27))
 (segment (start 167.005 82.58) (end 168.215002 82.58) (width 1) (layer B.Cu) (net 27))
 (segment (start 162.06363 86.36) (end 159.385 89.03863) (width 1.5) (layer F.Cu) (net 27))
 (segment (start 163.195 86.36) (end 162.06363 86.36) (width 1.5) (layer F.Cu) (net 27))
 (segment (start 159.385 89.03863) (end 159.385 102.235) (width 1.5) (layer F.Cu) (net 27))
 (segment (start 159.385 102.235) (end 161.29 104.14) (width 1.5) (layer F.Cu) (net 27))
 (segment (start 161.29 104.14) (end 163.195 104.14) (width 1.5) (layer F.Cu) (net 27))
 (segment (start 163.195 83.245) (end 163.86 82.58) (width 1) (layer B.Cu) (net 27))
 (segment (start 163.195 83.947) (end 163.195 83.245) (width 1) (layer B.Cu) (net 27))
 (segment (start 163.86 82.58) (end 163.195 82.58) (width 1) (layer B.Cu) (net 27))
 (segment (start 167.005 82.58) (end 163.86 82.58) (width 1) (layer B.Cu) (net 27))
 (segment (start 163.195 83.947) (end 163.195 86.36) (width 1) (layer B.Cu) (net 27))
 (segment (start 163.195 82.58) (end 163.195 83.947) (width 1) (layer B.Cu) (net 27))
 (segment (start 170.18 106.68) (end 172.72 106.68) (width 1.5) (layer F.Cu) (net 2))
 (segment (start 165.1 81.28) (end 165.1 81.28) (width 0.539) (layer F.Cu) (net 28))
 (via (at 165.1 81.28) (size 0.8) (drill 0.4) (layers F.Cu B.Cu) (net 28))
 (segment (start 165.1 81.28) (end 167.005 81.28) (width 1) (layer B.Cu) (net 28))
 (segment (start 155.829 71.501) (end 157.48 69.85) (width 0.539) (layer F.Cu) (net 28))
 (segment (start 155.829 74.454102) (end 155.829 71.501) (width 0.539) (layer F.Cu) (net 28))
 (segment (start 156.305397 74.930499) (end 155.829 74.454102) (width 0.539) (layer F.Cu) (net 28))
 (segment (start 164.465 88.9) (end 164.465 88.9) (width 0.539) (layer F.Cu) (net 28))
 (via (at 164.465 88.9) (size 0.8) (drill 0.4) (layers F.Cu B.Cu) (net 28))
 (segment (start 170.18 86.36) (end 165.1 81.28) (width 1) (layer F.Cu) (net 28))
 (segment (start 165.1 81.28) (end 165.1 80.01) (width 1) (layer F.Cu) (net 28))
 (segment (start 165.1 80.01) (end 163.449 78.359) (width 1) (layer F.Cu) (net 28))
 (segment (start 163.449 78.359) (end 163.449 78.359) (width 1) (layer F.Cu) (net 28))
 (via (at 163.449 78.359) (size 0.8) (drill 0.4) (layers F.Cu B.Cu) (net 28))
 (segment (start 164.846 78.359) (end 167.005 76.2) (width 1) (layer B.Cu) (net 28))
 (segment (start 163.449 78.359) (end 164.846 78.359) (width 1) (layer B.Cu) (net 28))
 (segment (start 167.64 88.9) (end 170.18 86.36) (width 1) (layer F.Cu) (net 28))
 (segment (start 164.465 88.9) (end 167.64 88.9) (width 1) (layer F.Cu) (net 28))
 (segment (start 156.306395 74.929501) (end 156.305397 74.930499) (width 0.539) (layer F.Cu) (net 28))
 (segment (start 165.734501 74.929501) (end 156.306395 74.929501) (width 0.539) (layer F.Cu) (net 28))
 (segment (start 167.005 76.2) (end 165.734501 74.929501) (width 0.539) (layer F.Cu) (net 28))
 (segment (start 170.18 104.14) (end 172.72 104.14) (width 1.5) (layer F.Cu) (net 4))
 (segment (start 154.94 78.74) (end 157.48 78.74) (width 1.5) (layer F.Cu) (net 5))
 (segment (start 170.18 101.6) (end 172.72 101.6) (width 1.5) (layer F.Cu) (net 6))
 (segment (start 154.94 81.28) (end 157.48 81.28) (width 1.5) (layer F.Cu) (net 7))
 (segment (start 170.18 99.06) (end 172.72 99.06) (width 1.5) (layer F.Cu) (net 8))
 (segment (start 154.94 83.82) (end 157.48 83.82) (width 1.5) (layer F.Cu) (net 9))
 (segment (start 170.18 96.52) (end 172.72 96.52) (width 1.5) (layer F.Cu) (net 10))
 (segment (start 154.94 86.36) (end 157.48 86.36) (width 1.5) (layer F.Cu) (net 11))
 (segment (start 170.18 88.9) (end 172.72 88.9) (width 1.5) (layer F.Cu) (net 12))
 (segment (start 171.45 92.71) (end 169.545 92.71) (width 0.54) (layer F.Cu) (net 12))
 (segment (start 172.72 93.98) (end 171.45 92.71) (width 0.54) (layer F.Cu) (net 12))
 (segment (start 169.380001 89.699999) (end 170.18 88.9) (width 0.54) (layer F.Cu) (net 12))
 (segment (start 168.909999 90.170001) (end 169.380001 89.699999) (width 0.54) (layer F.Cu) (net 12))
 (segment (start 168.909999 92.074999) (end 168.909999 90.170001) (width 0.54) (layer F.Cu) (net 12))
 (segment (start 169.545 92.71) (end 168.909999 92.074999) (width 0.54) (layer F.Cu) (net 12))
 (segment (start 154.94 88.9) (end 157.48 88.9) (width 1.5) (layer F.Cu) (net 13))
 (segment (start 170.18 91.44) (end 172.72 91.44) (width 1.5) (layer F.Cu) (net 14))
 (segment (start 154.94 91.44) (end 157.48 91.44) (width 1.5) (layer F.Cu) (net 15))
 (segment (start 154.94 93.98) (end 157.48 93.98) (width 1.5) (layer F.Cu) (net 16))
 (segment (start 171.920001 87.159999) (end 172.72 86.36) (width 0.54) (layer B.Cu) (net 17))
 (segment (start 171.45 87.63) (end 171.920001 87.159999) (width 0.54) (layer B.Cu) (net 17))
 (segment (start 171.45 92.71) (end 171.45 87.63) (width 0.54) (layer B.Cu) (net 17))
 (segment (start 170.18 93.98) (end 171.45 92.71) (width 0.54) (layer B.Cu) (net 17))
 (segment (start 154.94 96.52) (end 157.48 96.52) (width 1.5) (layer F.Cu) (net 18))
 (segment (start 170.18 83.82) (end 172.72 83.82) (width 1.5) (layer F.Cu) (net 19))
 (segment (start 154.94 99.06) (end 157.48 99.06) (width 1.5) (layer F.Cu) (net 20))
 (segment (start 170.18 81.28) (end 172.72 81.28) (width 1.5) (layer F.Cu) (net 21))
 (segment (start 154.94 101.6) (end 157.48 101.6) (width 1.5) (layer F.Cu) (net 22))
 (segment (start 154.94 104.14) (end 157.48 104.14) (width 1.5) (layer F.Cu) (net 24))
 (segment (start 157.48 73.66) (end 163.83 73.66) (width 1) (layer F.Cu) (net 1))
 (segment (start 165.1 72.39) (end 165.1 69.85) (width 1) (layer F.Cu) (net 1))
 (segment (start 163.83 73.66) (end 165.1 72.39) (width 1) (layer F.Cu) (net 1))
 (segment (start 163.195 99.06) (end 161.29 99.06) (width 1) (layer B.Cu) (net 1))
 (segment (start 161.29 99.06) (end 161.29 99.06) (width 1) (layer B.Cu) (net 1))
 (via (at 161.29 99.06) (size 0.8) (drill 0.4) (layers F.Cu B.Cu) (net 1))
 (segment (start 161.29 95.885) (end 163.195 93.98) (width 1) (layer F.Cu) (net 1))
 (segment (start 161.29 99.06) (end 161.29 95.885) (width 1) (layer F.Cu) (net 1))
 (segment (start 159.385 77.47) (end 159.385 77.47) (width 0.539) (layer B.Cu) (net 1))
 (via (at 159.385 77.47) (size 0.8) (drill 0.4) (layers F.Cu B.Cu) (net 1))
 (segment (start 159.385 82.55) (end 159.385 82.55) (width 0.539) (layer F.Cu) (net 1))
 (via (at 159.385 82.55) (size 0.8) (drill 0.4) (layers F.Cu B.Cu) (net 1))
 (segment (start 159.385 75.565) (end 157.48 73.66) (width 1) (layer B.Cu) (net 1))
 (segment (start 159.385 77.47) (end 159.385 75.565) (width 1) (layer B.Cu) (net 1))
 (segment (start 159.385 90.17) (end 163.195 93.98) (width 1) (layer B.Cu) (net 1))
 (segment (start 159.385 82.55) (end 159.385 90.17) (width 1) (layer B.Cu) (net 1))
 (segment (start 159.385 82.55) (end 159.385 77.47) (width 1) (layer F.Cu) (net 1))
 (segment (start 161.85501 83.88999) (end 161.054999 84.690001) (width 1) (layer F.Cu) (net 3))
 (segment (start 161.85501 78.24294) (end 161.85501 83.88999) (width 1) (layer F.Cu) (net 3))
 (segment (start 159.81207 76.2) (end 161.85501 78.24294) (width 1) (layer F.Cu) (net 3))
 (segment (start 157.48 76.2) (end 159.81207 76.2) (width 1) (layer F.Cu) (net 3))
 (segment (start 161.054999 84.690001) (end 161.054999 84.690001) (width 1) (layer F.Cu) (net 3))
 (via (at 161.054999 84.690001) (size 0.8) (drill 0.4) (layers F.Cu B.Cu) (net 3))
 (segment (start 161.054999 84.690001) (end 161.054999 88.029999) (width 1) (layer B.Cu) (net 3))
 (segment (start 161.054999 88.029999) (end 161.925 88.9) (width 1) (layer B.Cu) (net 3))
 (segment (start 161.925 88.9) (end 163.18 88.9) (width 1) (layer B.Cu) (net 3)))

